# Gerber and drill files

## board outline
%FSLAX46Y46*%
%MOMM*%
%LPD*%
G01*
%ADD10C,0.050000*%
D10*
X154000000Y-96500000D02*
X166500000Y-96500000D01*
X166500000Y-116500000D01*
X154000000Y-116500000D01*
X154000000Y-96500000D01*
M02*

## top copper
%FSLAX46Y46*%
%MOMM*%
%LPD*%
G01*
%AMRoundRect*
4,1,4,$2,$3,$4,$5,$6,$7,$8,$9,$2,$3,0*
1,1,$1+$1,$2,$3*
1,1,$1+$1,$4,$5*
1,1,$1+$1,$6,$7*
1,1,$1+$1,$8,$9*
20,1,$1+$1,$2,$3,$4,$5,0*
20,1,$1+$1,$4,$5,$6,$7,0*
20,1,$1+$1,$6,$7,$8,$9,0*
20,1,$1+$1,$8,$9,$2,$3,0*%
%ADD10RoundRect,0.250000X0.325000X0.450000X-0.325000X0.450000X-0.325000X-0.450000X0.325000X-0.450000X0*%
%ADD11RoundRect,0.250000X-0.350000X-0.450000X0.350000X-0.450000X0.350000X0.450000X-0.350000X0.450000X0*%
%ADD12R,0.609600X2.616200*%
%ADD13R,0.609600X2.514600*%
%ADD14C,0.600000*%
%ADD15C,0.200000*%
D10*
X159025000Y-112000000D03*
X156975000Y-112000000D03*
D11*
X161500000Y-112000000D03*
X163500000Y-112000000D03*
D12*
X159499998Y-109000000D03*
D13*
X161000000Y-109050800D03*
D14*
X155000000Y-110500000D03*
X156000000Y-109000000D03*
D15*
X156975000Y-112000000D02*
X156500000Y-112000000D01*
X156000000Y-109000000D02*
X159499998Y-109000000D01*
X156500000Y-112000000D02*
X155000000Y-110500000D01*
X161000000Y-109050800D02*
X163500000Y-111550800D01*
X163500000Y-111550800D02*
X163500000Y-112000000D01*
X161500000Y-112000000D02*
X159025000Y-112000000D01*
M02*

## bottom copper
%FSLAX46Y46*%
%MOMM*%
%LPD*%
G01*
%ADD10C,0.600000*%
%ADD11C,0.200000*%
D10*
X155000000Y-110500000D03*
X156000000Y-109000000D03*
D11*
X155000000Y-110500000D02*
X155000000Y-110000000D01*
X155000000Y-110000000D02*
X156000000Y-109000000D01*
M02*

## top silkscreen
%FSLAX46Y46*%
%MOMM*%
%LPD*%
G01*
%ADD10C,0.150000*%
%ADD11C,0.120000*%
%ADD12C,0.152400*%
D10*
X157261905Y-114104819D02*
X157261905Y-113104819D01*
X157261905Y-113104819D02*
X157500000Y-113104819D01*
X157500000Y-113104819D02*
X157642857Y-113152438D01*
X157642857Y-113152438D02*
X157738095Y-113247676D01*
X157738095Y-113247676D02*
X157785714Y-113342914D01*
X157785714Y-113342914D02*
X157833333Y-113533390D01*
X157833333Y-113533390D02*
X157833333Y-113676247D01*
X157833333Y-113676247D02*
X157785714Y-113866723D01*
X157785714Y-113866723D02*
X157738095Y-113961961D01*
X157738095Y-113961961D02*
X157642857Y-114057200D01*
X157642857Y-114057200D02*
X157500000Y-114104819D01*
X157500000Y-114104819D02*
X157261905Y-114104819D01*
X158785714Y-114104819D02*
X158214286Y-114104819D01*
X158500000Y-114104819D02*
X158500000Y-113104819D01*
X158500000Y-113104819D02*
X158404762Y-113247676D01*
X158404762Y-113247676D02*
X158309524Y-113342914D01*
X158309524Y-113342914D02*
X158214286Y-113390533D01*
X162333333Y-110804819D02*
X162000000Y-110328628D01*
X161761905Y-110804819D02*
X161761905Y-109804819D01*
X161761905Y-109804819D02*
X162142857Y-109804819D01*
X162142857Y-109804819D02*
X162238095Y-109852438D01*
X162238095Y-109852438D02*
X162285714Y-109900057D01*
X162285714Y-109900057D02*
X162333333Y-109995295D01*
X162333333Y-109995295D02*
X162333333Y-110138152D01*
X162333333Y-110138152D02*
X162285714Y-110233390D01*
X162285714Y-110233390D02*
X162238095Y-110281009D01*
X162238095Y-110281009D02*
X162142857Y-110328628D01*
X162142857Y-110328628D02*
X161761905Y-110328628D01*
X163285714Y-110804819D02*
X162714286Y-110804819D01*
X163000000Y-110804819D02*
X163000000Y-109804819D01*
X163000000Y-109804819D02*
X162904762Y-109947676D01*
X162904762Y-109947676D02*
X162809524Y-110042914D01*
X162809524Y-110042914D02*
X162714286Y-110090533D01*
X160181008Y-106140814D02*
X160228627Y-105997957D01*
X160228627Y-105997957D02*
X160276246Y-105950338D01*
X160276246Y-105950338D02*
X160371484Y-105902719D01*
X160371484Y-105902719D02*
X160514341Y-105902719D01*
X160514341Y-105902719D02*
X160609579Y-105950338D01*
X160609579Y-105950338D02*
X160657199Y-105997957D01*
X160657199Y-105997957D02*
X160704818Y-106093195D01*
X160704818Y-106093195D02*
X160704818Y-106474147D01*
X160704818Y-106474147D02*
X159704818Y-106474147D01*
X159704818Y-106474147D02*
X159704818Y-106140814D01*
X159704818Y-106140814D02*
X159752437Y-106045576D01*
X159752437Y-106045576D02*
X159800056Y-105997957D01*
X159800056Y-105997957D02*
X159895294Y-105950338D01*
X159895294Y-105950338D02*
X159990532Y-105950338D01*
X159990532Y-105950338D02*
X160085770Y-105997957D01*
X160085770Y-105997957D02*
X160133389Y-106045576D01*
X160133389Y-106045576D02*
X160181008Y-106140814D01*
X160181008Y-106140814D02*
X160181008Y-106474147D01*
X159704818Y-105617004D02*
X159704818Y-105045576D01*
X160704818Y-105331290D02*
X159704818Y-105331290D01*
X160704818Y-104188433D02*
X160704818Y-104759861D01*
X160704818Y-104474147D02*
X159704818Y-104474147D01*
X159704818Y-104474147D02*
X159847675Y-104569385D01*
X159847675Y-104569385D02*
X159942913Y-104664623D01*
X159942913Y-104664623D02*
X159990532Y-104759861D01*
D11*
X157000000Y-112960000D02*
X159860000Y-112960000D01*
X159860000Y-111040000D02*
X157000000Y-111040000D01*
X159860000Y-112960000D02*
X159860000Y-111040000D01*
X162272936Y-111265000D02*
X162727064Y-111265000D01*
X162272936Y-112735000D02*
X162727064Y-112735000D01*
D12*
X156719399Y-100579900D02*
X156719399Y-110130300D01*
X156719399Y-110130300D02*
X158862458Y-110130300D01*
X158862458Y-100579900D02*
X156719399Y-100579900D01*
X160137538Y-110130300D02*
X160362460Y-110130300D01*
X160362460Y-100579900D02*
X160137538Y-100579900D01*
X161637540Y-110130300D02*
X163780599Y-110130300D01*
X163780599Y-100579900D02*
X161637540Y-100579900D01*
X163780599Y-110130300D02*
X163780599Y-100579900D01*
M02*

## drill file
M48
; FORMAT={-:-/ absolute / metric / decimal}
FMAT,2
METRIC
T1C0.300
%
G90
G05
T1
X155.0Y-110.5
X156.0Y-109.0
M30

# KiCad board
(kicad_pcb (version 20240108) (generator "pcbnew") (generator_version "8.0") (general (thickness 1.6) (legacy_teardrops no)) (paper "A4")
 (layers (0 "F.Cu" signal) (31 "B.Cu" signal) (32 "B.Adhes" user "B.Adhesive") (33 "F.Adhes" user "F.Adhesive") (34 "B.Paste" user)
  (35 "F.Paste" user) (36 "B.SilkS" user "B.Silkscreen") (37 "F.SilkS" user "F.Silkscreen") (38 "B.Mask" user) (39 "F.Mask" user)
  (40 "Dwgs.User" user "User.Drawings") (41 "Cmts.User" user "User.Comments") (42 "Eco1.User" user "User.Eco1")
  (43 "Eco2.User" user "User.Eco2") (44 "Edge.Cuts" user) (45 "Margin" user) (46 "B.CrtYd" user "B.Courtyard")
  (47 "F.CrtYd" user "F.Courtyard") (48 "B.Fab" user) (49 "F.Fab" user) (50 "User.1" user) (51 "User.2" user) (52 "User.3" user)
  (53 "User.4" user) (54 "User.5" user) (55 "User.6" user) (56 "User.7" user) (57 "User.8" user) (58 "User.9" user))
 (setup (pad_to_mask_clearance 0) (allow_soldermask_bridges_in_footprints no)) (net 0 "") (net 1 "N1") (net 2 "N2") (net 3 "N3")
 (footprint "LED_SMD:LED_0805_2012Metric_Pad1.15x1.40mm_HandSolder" (layer "F.Cu") (at 158 112 180)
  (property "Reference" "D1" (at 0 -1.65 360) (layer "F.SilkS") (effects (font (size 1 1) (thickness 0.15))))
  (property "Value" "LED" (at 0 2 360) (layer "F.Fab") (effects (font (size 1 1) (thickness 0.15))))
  (fp_line (start 1 -0.96) (end -1.86 -0.96) (stroke (width 0.12) (type solid)) (layer "F.SilkS"))
  (fp_line (start -1.86 0.96) (end 1 0.96) (stroke (width 0.12) (type solid)) (layer "F.SilkS"))
  (fp_line (start -1.86 -0.96) (end -1.86 0.96) (stroke (width 0.12) (type solid)) (layer "F.SilkS"))
  (pad "1" smd roundrect (at -1.025 0 180) (size 1.15 1.4) (layers "F.Cu" "F.Paste" "F.Mask") (roundrect_rratio 0.217391) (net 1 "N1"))
  (pad "2" smd roundrect (at 1.025 0 180) (size 1.15 1.4) (layers "F.Cu" "F.Paste" "F.Mask") (roundrect_rratio 0.217391) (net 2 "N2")))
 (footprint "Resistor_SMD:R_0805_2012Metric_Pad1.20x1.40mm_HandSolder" (layer "F.Cu") (at 162.5 112)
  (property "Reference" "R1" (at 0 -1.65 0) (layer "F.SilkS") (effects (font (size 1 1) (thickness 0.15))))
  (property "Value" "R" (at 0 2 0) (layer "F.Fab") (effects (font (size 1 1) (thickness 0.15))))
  (fp_line (start -0.227064 -0.735) (end 0.227064 -0.735) (stroke (width 0.12) (type solid)) (layer "F.SilkS"))
  (fp_line (start -0.227064 0.735) (end 0.227064 0.735) (stroke (width 0.12) (type solid)) (layer "F.SilkS"))
  (pad "1" smd roundrect (at -1 0) (size 1.2 1.4) (layers "F.Cu" "F.Paste" "F.Mask") (roundrect_rratio 0.208333) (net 1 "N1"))
  (pad "2" smd roundrect (at 1 0) (size 1.2 1.4) (layers "F.Cu" "F.Paste" "F.Mask") (roundrect_rratio 0.208333) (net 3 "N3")))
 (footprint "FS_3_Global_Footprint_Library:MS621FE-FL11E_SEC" (layer "F.Cu") (at 160.249999 105.3551 90)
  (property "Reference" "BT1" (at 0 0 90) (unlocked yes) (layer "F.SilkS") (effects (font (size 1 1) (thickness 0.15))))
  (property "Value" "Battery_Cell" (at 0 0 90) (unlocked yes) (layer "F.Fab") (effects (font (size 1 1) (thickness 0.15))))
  (fp_line (start 4.7752 -3.5306) (end -4.7752 -3.5306) (stroke (width 0.1524) (type solid)) (layer "F.SilkS"))
  (fp_line (start -4.7752 -3.5306) (end -4.7752 -1.387541) (stroke (width 0.1524) (type solid)) (layer "F.SilkS"))
  (fp_line (start 4.7752 -1.387541) (end 4.7752 -3.5306) (stroke (width 0.1524) (type solid)) (layer "F.SilkS"))
  (fp_line (start -4.7752 -0.112461) (end -4.7752 0.112461) (stroke (width 0.1524) (type solid)) (layer "F.SilkS"))
  (fp_line (start 4.7752 0.112461) (end 4.7752 -0.112461) (stroke (width 0.1524) (type solid)) (layer "F.SilkS"))
  (fp_line (start -4.7752 1.387541) (end -4.7752 3.5306) (stroke (width 0.1524) (type solid)) (layer "F.SilkS"))
  (fp_line (start 4.7752 3.5306) (end 4.7752 1.387541) (stroke (width 0.1524) (type solid)) (layer "F.SilkS"))
  (fp_line (start -4.7752 3.5306) (end 4.7752 3.5306) (stroke (width 0.1524) (type solid)) (layer "F.SilkS"))
  (pad "1" smd rect (at -3.6449 -0.750001 90) (size 2.6162 0.6096) (layers "F.Cu" "F.Paste" "F.Mask") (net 2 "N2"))
  (pad "2" smd rect (at -3.6957 0.750001 90) (size 2.5146 0.6096) (layers "F.Cu" "F.Paste" "F.Mask") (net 3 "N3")))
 (gr_rect (start 154 96.5) (end 166.5 116.5) (stroke (width 0.05) (type default)) (fill none) (layer "Edge.Cuts"))
 (segment (start 156.975 112) (end 156.5 112) (width 0.2) (layer "F.Cu") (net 2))
 (segment (start 156 109) (end 159.499998 109) (width 0.2) (layer "F.Cu") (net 2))
 (segment (start 156.5 112) (end 155 110.5) (width 0.2) (layer "F.Cu") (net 2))
 (via (at 155 110.5) (size 0.6) (drill 0.3) (layers "F.Cu" "B.Cu") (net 2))
 (via (at 156 109) (size 0.6) (drill 0.3) (layers "F.Cu" "B.Cu") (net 2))
 (segment (start 155 110.5) (end 155 110) (width 0.2) (layer "B.Cu") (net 2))
 (segment (start 155 110) (end 156 109) (width 0.2) (layer "B.Cu") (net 2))
 (segment (start 161 109.0508) (end 163.5 111.5508) (width 0.2) (layer "F.Cu") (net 3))
 (segment (start 163.5 111.5508) (end 163.5 112) (width 0.2) (layer "F.Cu") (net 3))
 (segment (start 161.5 112) (end 159.025 112) (width 0.2) (layer "F.Cu") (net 1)))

